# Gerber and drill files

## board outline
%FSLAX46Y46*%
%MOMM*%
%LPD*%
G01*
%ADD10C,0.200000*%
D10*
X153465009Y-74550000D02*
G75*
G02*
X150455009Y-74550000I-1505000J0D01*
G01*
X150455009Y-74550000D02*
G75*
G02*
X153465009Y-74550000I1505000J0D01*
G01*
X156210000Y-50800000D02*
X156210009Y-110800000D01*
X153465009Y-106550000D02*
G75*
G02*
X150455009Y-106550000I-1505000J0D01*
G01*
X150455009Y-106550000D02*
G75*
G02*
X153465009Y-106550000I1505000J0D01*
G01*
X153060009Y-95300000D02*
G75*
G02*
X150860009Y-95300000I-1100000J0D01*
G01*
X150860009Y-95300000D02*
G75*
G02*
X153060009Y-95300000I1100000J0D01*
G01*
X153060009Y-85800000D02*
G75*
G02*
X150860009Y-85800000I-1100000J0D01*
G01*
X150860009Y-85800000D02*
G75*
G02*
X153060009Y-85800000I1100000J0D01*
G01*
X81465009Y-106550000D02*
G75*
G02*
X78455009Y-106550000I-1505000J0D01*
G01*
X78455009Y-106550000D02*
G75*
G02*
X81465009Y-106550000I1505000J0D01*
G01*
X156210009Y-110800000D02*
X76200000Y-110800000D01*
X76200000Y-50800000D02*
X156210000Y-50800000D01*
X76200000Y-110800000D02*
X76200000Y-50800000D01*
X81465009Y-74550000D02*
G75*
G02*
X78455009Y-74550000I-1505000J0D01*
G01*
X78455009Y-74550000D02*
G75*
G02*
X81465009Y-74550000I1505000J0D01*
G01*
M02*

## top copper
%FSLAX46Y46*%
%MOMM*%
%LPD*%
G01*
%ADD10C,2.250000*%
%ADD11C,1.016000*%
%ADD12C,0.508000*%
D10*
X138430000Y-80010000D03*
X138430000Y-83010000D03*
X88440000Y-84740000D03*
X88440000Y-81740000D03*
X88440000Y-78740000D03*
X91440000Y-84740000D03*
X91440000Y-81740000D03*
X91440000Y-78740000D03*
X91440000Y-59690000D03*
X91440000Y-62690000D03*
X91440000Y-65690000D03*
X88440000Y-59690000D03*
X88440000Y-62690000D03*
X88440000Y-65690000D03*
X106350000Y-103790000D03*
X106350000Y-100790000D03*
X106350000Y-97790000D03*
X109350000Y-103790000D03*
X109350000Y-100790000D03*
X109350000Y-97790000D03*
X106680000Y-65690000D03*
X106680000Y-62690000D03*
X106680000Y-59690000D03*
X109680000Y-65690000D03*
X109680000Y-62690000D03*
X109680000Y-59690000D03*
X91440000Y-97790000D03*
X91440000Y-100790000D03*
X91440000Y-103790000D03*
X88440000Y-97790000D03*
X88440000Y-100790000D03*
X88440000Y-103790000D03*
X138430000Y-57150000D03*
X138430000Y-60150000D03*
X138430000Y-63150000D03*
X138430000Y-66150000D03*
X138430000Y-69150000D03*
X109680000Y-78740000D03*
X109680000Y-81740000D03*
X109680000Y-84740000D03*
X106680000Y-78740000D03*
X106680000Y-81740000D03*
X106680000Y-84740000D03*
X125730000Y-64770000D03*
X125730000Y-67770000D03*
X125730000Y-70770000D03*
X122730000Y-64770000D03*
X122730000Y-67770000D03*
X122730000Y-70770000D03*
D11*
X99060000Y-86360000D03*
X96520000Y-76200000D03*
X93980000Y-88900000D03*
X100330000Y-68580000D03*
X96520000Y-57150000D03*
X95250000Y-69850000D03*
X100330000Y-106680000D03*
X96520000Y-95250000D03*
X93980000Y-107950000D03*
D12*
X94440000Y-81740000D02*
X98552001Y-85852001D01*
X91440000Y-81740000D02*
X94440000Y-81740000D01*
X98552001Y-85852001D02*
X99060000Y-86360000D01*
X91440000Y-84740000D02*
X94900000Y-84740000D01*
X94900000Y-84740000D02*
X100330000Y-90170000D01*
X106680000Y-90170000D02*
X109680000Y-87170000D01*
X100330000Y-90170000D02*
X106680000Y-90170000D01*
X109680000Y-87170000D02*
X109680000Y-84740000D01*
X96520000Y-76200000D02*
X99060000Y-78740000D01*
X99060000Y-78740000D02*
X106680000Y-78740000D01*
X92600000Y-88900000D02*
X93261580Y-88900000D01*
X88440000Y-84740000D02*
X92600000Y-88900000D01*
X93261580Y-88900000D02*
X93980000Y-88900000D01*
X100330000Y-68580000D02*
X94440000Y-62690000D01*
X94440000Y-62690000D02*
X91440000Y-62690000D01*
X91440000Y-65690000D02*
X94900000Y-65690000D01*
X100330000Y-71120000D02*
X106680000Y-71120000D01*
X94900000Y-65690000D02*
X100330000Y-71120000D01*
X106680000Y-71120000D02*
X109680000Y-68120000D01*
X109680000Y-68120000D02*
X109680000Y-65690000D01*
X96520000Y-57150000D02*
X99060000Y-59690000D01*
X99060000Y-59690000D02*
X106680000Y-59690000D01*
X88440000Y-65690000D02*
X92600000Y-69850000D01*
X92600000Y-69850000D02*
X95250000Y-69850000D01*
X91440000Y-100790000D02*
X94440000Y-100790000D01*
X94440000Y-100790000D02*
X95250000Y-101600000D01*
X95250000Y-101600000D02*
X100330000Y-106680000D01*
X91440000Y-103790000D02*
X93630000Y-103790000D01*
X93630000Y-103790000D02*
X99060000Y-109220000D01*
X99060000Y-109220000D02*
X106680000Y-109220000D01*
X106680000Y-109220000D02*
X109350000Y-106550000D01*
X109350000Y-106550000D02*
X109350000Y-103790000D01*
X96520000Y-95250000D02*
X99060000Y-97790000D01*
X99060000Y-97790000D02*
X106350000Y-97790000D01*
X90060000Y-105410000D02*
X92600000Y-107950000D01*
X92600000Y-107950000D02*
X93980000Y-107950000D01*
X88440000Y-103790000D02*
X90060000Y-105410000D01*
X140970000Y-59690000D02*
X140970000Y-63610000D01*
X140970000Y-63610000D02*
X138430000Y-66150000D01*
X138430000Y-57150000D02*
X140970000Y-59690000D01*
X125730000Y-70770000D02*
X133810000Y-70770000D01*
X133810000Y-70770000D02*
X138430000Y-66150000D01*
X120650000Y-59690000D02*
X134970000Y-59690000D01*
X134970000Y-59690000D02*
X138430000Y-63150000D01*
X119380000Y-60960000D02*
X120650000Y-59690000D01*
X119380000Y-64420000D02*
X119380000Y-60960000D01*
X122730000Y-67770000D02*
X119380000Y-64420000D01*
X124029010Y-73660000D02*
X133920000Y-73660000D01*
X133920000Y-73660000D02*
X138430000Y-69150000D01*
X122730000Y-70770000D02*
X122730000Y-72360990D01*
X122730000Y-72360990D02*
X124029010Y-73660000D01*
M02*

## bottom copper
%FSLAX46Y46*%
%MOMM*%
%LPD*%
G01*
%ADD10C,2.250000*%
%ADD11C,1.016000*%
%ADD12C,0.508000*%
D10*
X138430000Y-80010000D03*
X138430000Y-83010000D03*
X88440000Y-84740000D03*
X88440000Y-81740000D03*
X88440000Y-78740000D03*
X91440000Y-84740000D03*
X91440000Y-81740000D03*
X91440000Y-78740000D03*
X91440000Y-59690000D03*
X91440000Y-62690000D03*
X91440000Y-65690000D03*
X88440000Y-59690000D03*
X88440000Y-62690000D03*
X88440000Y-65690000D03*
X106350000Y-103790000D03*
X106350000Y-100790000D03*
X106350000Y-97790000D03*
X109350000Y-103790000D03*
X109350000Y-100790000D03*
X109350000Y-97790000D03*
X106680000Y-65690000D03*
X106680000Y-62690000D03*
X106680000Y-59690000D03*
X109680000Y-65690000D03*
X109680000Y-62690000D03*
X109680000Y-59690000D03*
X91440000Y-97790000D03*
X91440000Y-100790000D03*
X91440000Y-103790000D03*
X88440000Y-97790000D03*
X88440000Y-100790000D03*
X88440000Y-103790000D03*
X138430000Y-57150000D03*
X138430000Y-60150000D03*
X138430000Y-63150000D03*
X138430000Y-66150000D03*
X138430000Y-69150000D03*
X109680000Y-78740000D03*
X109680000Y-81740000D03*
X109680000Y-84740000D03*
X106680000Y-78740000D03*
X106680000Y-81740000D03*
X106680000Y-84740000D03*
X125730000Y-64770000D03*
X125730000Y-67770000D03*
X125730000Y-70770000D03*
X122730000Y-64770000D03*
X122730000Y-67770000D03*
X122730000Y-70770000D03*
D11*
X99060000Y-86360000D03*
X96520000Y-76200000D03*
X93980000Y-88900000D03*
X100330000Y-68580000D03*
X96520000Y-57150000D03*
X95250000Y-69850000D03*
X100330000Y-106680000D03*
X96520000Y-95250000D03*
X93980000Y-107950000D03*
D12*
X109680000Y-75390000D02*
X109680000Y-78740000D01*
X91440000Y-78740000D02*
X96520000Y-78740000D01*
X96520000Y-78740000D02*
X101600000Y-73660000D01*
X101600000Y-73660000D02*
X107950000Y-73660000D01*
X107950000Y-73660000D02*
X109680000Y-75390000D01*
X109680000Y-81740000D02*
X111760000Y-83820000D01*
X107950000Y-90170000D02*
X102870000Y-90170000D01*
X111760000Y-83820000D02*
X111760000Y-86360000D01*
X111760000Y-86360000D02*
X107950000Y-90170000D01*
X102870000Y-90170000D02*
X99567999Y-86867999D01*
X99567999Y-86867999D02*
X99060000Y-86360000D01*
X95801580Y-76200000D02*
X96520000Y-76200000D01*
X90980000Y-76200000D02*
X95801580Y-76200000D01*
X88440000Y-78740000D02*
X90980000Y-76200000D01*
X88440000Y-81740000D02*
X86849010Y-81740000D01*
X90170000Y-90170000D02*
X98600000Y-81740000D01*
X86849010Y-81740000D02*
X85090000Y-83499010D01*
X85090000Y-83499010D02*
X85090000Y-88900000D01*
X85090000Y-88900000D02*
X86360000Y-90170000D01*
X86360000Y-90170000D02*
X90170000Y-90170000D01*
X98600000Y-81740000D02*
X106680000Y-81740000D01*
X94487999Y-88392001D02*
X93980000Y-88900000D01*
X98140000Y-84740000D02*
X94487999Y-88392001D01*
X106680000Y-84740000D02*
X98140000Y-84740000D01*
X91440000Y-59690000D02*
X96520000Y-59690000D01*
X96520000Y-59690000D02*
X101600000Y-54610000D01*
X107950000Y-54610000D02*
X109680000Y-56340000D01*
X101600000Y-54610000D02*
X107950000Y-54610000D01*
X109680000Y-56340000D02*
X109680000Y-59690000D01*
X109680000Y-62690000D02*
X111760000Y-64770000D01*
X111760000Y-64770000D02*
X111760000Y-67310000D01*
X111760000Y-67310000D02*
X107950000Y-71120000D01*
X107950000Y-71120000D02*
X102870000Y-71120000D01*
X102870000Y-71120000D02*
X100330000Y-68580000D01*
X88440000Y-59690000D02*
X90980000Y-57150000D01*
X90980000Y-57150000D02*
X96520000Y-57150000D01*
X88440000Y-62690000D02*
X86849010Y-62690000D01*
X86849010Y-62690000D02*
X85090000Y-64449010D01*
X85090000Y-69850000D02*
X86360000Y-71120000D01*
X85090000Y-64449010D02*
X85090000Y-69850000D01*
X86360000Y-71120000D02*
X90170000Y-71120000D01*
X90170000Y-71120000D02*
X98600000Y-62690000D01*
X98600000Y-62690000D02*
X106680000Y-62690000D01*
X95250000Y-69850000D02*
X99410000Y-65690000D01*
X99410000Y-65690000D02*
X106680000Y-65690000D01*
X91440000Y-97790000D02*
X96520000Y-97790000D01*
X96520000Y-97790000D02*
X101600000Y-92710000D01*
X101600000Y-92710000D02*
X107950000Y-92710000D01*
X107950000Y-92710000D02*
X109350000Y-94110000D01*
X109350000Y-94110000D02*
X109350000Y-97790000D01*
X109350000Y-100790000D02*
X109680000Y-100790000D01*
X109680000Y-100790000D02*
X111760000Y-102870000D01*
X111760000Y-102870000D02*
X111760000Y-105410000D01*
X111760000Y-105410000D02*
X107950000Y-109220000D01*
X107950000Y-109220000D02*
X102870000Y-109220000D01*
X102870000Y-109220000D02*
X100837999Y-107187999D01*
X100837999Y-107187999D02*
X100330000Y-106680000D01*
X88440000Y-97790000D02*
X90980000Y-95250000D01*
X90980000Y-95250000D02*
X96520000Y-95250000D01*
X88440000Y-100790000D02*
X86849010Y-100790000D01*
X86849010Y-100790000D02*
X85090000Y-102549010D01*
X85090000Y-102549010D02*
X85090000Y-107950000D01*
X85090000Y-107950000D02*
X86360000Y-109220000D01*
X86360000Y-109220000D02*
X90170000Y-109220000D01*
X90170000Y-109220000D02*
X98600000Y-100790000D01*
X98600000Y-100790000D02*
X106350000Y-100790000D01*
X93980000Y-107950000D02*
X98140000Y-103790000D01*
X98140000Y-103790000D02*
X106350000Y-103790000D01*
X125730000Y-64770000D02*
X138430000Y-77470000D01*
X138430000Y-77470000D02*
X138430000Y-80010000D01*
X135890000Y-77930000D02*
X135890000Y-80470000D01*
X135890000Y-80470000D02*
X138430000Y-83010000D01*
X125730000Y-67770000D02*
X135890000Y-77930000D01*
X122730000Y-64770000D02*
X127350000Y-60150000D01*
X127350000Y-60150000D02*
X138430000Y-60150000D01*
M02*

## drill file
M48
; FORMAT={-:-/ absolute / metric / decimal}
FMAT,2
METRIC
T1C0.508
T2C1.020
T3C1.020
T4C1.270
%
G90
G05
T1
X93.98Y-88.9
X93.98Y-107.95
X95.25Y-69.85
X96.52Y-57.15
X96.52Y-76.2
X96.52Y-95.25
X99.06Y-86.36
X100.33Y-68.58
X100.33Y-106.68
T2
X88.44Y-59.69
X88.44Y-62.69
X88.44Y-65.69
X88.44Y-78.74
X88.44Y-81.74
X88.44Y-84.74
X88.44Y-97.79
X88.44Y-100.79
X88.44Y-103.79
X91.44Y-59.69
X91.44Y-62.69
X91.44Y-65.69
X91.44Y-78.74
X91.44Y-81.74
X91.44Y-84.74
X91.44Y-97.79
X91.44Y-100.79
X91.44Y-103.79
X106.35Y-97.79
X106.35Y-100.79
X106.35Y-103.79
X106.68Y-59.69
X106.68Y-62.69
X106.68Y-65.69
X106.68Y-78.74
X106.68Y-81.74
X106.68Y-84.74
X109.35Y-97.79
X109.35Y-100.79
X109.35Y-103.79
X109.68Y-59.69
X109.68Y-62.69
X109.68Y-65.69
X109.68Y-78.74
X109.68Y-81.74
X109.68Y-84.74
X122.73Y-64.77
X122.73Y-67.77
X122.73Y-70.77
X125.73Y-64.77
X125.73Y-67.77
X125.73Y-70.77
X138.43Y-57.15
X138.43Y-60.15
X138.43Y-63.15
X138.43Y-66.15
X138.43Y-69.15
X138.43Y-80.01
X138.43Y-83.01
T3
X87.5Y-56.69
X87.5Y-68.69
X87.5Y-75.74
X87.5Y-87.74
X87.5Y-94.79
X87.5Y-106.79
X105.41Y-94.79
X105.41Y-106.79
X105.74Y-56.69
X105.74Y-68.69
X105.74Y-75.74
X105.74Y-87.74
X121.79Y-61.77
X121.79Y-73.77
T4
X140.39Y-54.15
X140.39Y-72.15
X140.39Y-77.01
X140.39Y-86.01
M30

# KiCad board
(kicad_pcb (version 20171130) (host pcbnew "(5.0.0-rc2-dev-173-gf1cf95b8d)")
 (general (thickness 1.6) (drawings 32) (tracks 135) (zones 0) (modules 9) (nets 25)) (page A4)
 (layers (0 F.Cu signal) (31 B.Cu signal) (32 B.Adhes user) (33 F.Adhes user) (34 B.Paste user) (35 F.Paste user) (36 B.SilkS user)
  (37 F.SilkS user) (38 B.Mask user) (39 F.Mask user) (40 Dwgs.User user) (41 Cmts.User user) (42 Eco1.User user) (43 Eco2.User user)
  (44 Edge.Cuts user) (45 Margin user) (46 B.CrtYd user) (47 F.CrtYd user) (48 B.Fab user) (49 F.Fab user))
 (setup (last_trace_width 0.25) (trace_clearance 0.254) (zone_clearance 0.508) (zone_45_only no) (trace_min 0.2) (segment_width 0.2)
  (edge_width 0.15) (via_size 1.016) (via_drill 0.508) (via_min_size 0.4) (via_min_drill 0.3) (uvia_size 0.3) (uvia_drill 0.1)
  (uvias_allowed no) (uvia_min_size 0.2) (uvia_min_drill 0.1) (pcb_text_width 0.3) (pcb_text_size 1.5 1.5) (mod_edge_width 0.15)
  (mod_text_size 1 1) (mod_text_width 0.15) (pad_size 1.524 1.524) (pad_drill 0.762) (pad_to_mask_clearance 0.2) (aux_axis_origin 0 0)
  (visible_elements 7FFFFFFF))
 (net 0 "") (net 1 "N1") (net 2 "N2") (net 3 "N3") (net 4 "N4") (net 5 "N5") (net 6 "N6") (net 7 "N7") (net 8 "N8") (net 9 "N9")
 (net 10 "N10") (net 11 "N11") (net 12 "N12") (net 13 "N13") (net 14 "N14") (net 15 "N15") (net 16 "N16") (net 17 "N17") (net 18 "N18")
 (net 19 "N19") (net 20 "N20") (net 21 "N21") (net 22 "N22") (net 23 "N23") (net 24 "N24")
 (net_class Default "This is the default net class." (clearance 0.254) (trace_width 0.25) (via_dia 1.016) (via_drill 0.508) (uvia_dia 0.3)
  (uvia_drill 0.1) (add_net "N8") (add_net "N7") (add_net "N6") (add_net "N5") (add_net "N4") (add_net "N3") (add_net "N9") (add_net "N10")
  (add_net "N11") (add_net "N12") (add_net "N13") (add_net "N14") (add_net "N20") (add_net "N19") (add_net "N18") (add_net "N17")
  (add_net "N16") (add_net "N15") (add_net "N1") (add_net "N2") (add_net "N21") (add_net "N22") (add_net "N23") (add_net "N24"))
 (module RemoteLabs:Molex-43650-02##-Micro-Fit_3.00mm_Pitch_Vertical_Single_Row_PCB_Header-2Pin (layer F.Cu) (at 138.43 80.01 90)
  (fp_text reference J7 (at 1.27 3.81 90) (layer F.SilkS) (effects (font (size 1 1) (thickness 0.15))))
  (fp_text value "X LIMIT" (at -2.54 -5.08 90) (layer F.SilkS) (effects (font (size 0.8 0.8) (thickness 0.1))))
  (pad 1 thru_hole circle (at 0 0 90) (size 2.25 2.25) (drill 1.02) (layers *.Cu *.Mask F.SilkS) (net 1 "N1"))
  (pad 2 thru_hole circle (at -3 0 90) (size 2.25 2.25) (drill 1.02) (layers *.Cu *.Mask F.SilkS) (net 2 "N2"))
  (pad "" np_thru_hole circle (at 3 1.96 90) (size 1.27 1.27) (drill 1.27) (layers *.Cu *.Mask F.SilkS))
  (pad "" np_thru_hole circle (at -6 1.96 90) (size 1.27 1.27) (drill 1.27) (layers *.Cu *.Mask F.SilkS)))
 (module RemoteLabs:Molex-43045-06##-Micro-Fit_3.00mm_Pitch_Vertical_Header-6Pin (layer F.Cu) (at 91.44 78.74 90)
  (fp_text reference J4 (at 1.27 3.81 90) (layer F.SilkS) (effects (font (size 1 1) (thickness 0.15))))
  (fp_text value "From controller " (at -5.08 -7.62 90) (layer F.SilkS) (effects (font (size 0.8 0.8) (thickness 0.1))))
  (pad 6 thru_hole circle (at -6 -3 90) (size 2.25 2.25) (drill 1.02) (layers *.Cu *.Mask F.SilkS) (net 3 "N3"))
  (pad 5 thru_hole circle (at -3 -3 90) (size 2.25 2.25) (drill 1.02) (layers *.Cu *.Mask F.SilkS) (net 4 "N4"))
  (pad 4 thru_hole circle (at 0 -3 90) (size 2.25 2.25) (drill 1.02) (layers *.Cu *.Mask F.SilkS) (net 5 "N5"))
  (pad 3 thru_hole circle (at -6 0 90) (size 2.25 2.25) (drill 1.02) (layers *.Cu *.Mask F.SilkS) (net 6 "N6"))
  (pad 2 thru_hole circle (at -3 0 90) (size 2.25 2.25) (drill 1.02) (layers *.Cu *.Mask F.SilkS) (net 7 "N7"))
  (pad 1 thru_hole circle (at 0 0 90) (size 2.25 2.25) (drill 1.02) (layers *.Cu *.Mask F.SilkS) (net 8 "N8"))
  (pad "" np_thru_hole circle (at -9 -3.94 90) (size 1.02 1.02) (drill 1.02) (layers *.Cu *.Mask F.SilkS))
  (pad "" np_thru_hole circle (at 3 -3.94 90) (size 1.02 1.02) (drill 1.02) (layers *.Cu *.Mask F.SilkS)))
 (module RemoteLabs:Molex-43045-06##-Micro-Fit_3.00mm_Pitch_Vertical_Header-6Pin (layer F.Cu) (at 91.44 59.69 90)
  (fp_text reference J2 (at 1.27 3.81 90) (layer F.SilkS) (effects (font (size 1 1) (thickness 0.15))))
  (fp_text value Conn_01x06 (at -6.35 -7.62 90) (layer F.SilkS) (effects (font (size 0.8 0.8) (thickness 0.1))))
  (pad "" np_thru_hole circle (at 3 -3.94 90) (size 1.02 1.02) (drill 1.02) (layers *.Cu *.Mask F.SilkS))
  (pad "" np_thru_hole circle (at -9 -3.94 90) (size 1.02 1.02) (drill 1.02) (layers *.Cu *.Mask F.SilkS))
  (pad 1 thru_hole circle (at 0 0 90) (size 2.25 2.25) (drill 1.02) (layers *.Cu *.Mask F.SilkS) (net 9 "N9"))
  (pad 2 thru_hole circle (at -3 0 90) (size 2.25 2.25) (drill 1.02) (layers *.Cu *.Mask F.SilkS) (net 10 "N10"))
  (pad 3 thru_hole circle (at -6 0 90) (size 2.25 2.25) (drill 1.02) (layers *.Cu *.Mask F.SilkS) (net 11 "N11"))
  (pad 4 thru_hole circle (at 0 -3 90) (size 2.25 2.25) (drill 1.02) (layers *.Cu *.Mask F.SilkS) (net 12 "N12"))
  (pad 5 thru_hole circle (at -3 -3 90) (size 2.25 2.25) (drill 1.02) (layers *.Cu *.Mask F.SilkS) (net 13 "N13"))
  (pad 6 thru_hole circle (at -6 -3 90) (size 2.25 2.25) (drill 1.02) (layers *.Cu *.Mask F.SilkS) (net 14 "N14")))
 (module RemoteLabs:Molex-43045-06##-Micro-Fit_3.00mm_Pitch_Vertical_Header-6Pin (layer F.Cu) (at 109.35 97.79 90)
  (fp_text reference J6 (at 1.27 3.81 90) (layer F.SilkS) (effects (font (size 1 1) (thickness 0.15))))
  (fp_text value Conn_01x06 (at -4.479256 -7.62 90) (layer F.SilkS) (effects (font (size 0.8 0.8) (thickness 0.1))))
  (pad 6 thru_hole circle (at -6 -3 90) (size 2.25 2.25) (drill 1.02) (layers *.Cu *.Mask F.SilkS) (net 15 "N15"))
  (pad 5 thru_hole circle (at -3 -3 90) (size 2.25 2.25) (drill 1.02) (layers *.Cu *.Mask F.SilkS) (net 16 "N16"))
  (pad 4 thru_hole circle (at 0 -3 90) (size 2.25 2.25) (drill 1.02) (layers *.Cu *.Mask F.SilkS) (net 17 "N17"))
  (pad 3 thru_hole circle (at -6 0 90) (size 2.25 2.25) (drill 1.02) (layers *.Cu *.Mask F.SilkS) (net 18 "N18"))
  (pad 2 thru_hole circle (at -3 0 90) (size 2.25 2.25) (drill 1.02) (layers *.Cu *.Mask F.SilkS) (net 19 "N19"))
  (pad 1 thru_hole circle (at 0 0 90) (size 2.25 2.25) (drill 1.02) (layers *.Cu *.Mask F.SilkS) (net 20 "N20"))
  (pad "" np_thru_hole circle (at -9 -3.94 90) (size 1.02 1.02) (drill 1.02) (layers *.Cu *.Mask F.SilkS))
  (pad "" np_thru_hole circle (at 3 -3.94 90) (size 1.02 1.02) (drill 1.02) (layers *.Cu *.Mask F.SilkS)))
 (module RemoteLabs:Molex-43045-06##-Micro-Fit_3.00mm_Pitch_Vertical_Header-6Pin (layer F.Cu) (at 109.68 59.69 90)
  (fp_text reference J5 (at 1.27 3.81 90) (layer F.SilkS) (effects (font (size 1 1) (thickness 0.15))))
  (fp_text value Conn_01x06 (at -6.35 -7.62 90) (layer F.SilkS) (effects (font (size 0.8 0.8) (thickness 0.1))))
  (pad 6 thru_hole circle (at -6 -3 90) (size 2.25 2.25) (drill 1.02) (layers *.Cu *.Mask F.SilkS) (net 14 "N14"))
  (pad 5 thru_hole circle (at -3 -3 90) (size 2.25 2.25) (drill 1.02) (layers *.Cu *.Mask F.SilkS) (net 13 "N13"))
  (pad 4 thru_hole circle (at 0 -3 90) (size 2.25 2.25) (drill 1.02) (layers *.Cu *.Mask F.SilkS) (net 12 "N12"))
  (pad 3 thru_hole circle (at -6 0 90) (size 2.25 2.25) (drill 1.02) (layers *.Cu *.Mask F.SilkS) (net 11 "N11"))
  (pad 2 thru_hole circle (at -3 0 90) (size 2.25 2.25) (drill 1.02) (layers *.Cu *.Mask F.SilkS) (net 10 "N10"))
  (pad 1 thru_hole circle (at 0 0 90) (size 2.25 2.25) (drill 1.02) (layers *.Cu *.Mask F.SilkS) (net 9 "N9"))
  (pad "" np_thru_hole circle (at -9 -3.94 90) (size 1.02 1.02) (drill 1.02) (layers *.Cu *.Mask F.SilkS))
  (pad "" np_thru_hole circle (at 3 -3.94 90) (size 1.02 1.02) (drill 1.02) (layers *.Cu *.Mask F.SilkS)))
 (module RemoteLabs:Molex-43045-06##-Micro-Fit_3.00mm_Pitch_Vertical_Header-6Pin (layer F.Cu) (at 91.44 97.79 90)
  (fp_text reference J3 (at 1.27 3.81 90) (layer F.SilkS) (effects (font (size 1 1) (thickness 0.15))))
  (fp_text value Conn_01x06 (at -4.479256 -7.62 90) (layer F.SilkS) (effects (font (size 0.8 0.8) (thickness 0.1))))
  (pad "" np_thru_hole circle (at 3 -3.94 90) (size 1.02 1.02) (drill 1.02) (layers *.Cu *.Mask F.SilkS))
  (pad "" np_thru_hole circle (at -9 -3.94 90) (size 1.02 1.02) (drill 1.02) (layers *.Cu *.Mask F.SilkS))
  (pad 1 thru_hole circle (at 0 0 90) (size 2.25 2.25) (drill 1.02) (layers *.Cu *.Mask F.SilkS) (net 20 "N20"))
  (pad 2 thru_hole circle (at -3 0 90) (size 2.25 2.25) (drill 1.02) (layers *.Cu *.Mask F.SilkS) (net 19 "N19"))
  (pad 3 thru_hole circle (at -6 0 90) (size 2.25 2.25) (drill 1.02) (layers *.Cu *.Mask F.SilkS) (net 18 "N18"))
  (pad 4 thru_hole circle (at 0 -3 90) (size 2.25 2.25) (drill 1.02) (layers *.Cu *.Mask F.SilkS) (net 17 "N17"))
  (pad 5 thru_hole circle (at -3 -3 90) (size 2.25 2.25) (drill 1.02) (layers *.Cu *.Mask F.SilkS) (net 16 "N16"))
  (pad 6 thru_hole circle (at -6 -3 90) (size 2.25 2.25) (drill 1.02) (layers *.Cu *.Mask F.SilkS) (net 15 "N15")))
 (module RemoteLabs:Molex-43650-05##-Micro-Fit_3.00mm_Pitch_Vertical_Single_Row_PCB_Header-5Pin (layer F.Cu) (at 138.43 57.15 90)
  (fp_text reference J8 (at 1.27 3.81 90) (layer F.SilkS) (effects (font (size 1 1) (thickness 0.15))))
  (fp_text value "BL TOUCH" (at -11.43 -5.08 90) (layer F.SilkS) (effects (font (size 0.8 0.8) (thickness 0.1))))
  (pad 1 thru_hole circle (at 0 0 90) (size 2.25 2.25) (drill 1.02) (layers *.Cu *.Mask F.SilkS) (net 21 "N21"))
  (pad 2 thru_hole circle (at -3 0 90) (size 2.25 2.25) (drill 1.02) (layers *.Cu *.Mask F.SilkS) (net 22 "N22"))
  (pad 3 thru_hole circle (at -6 0 90) (size 2.25 2.25) (drill 1.02) (layers *.Cu *.Mask F.SilkS) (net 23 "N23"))
  (pad 4 thru_hole circle (at -9 0 90) (size 2.25 2.25) (drill 1.02) (layers *.Cu *.Mask F.SilkS) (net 21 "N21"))
  (pad 5 thru_hole circle (at -12 0 90) (size 2.25 2.25) (drill 1.02) (layers *.Cu *.Mask F.SilkS) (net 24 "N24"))
  (pad "" np_thru_hole circle (at 3 1.96 90) (size 1.27 1.27) (drill 1.27) (layers *.Cu *.Mask F.SilkS))
  (pad "" np_thru_hole circle (at -15 1.96 90) (size 1.27 1.27) (drill 1.27) (layers *.Cu *.Mask F.SilkS)))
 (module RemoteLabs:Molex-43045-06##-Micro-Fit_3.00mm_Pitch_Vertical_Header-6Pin (layer F.Cu) (at 109.68 78.74 90)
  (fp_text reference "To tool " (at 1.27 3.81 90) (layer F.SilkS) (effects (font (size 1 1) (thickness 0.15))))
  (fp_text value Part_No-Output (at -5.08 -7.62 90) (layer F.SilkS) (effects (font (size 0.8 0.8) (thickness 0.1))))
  (pad "" np_thru_hole circle (at 3 -3.94 90) (size 1.02 1.02) (drill 1.02) (layers *.Cu *.Mask F.SilkS))
  (pad "" np_thru_hole circle (at -9 -3.94 90) (size 1.02 1.02) (drill 1.02) (layers *.Cu *.Mask F.SilkS))
  (pad 1 thru_hole circle (at 0 0 90) (size 2.25 2.25) (drill 1.02) (layers *.Cu *.Mask F.SilkS) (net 8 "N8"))
  (pad 2 thru_hole circle (at -3 0 90) (size 2.25 2.25) (drill 1.02) (layers *.Cu *.Mask F.SilkS) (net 7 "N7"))
  (pad 3 thru_hole circle (at -6 0 90) (size 2.25 2.25) (drill 1.02) (layers *.Cu *.Mask F.SilkS) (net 6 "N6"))
  (pad 4 thru_hole circle (at 0 -3 90) (size 2.25 2.25) (drill 1.02) (layers *.Cu *.Mask F.SilkS) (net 5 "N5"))
  (pad 5 thru_hole circle (at -3 -3 90) (size 2.25 2.25) (drill 1.02) (layers *.Cu *.Mask F.SilkS) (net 4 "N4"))
  (pad 6 thru_hole circle (at -6 -3 90) (size 2.25 2.25) (drill 1.02) (layers *.Cu *.Mask F.SilkS) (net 3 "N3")))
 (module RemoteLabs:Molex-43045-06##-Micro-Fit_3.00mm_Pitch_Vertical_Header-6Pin (layer F.Cu) (at 125.73 64.77 90)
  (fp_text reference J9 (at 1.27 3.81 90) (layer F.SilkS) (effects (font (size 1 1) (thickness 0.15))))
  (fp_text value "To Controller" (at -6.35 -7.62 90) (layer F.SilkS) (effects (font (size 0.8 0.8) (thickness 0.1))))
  (pad "" np_thru_hole circle (at 3 -3.94 90) (size 1.02 1.02) (drill 1.02) (layers *.Cu *.Mask F.SilkS))
  (pad "" np_thru_hole circle (at -9 -3.94 90) (size 1.02 1.02) (drill 1.02) (layers *.Cu *.Mask F.SilkS))
  (pad 1 thru_hole circle (at 0 0 90) (size 2.25 2.25) (drill 1.02) (layers *.Cu *.Mask F.SilkS) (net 1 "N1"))
  (pad 2 thru_hole circle (at -3 0 90) (size 2.25 2.25) (drill 1.02) (layers *.Cu *.Mask F.SilkS) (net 2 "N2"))
  (pad 3 thru_hole circle (at -6 0 90) (size 2.25 2.25) (drill 1.02) (layers *.Cu *.Mask F.SilkS) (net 21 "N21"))
  (pad 4 thru_hole circle (at 0 -3 90) (size 2.25 2.25) (drill 1.02) (layers *.Cu *.Mask F.SilkS) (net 22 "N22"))
  (pad 5 thru_hole circle (at -3 -3 90) (size 2.25 2.25) (drill 1.02) (layers *.Cu *.Mask F.SilkS) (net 23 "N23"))
  (pad 6 thru_hole circle (at -6 -3 90) (size 2.25 2.25) (drill 1.02) (layers *.Cu *.Mask F.SilkS) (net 24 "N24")))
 (gr_circle (center 151.960009 74.55) (end 153.465009 74.55) (layer Edge.Cuts) (width 0.2))
 (gr_line (start 156.21 50.8) (end 156.210009 110.8) (layer Edge.Cuts) (width 0.2))
 (gr_circle (center 151.960009 106.55) (end 153.465009 106.55) (layer Edge.Cuts) (width 0.2))
 (gr_circle (center 151.960009 95.3) (end 153.060009 95.3) (layer Edge.Cuts) (width 0.2))
 (gr_circle (center 151.960009 85.8) (end 153.060009 85.8) (layer Edge.Cuts) (width 0.2))
 (gr_circle (center 79.960009 106.55) (end 81.465009 106.55) (layer Edge.Cuts) (width 0.2))
 (gr_line (start 156.210009 110.8) (end 76.2 110.8) (layer Edge.Cuts) (width 0.2))
 (gr_line (start 76.2 50.8) (end 156.21 50.8) (layer Edge.Cuts) (width 0.2))
 (gr_line (start 76.2 110.8) (end 76.2 50.8) (layer Edge.Cuts) (width 0.2))
 (gr_circle (center 79.960009 74.55) (end 81.465009 74.55) (layer Edge.Cuts) (width 0.2))
 (segment (start 109.68 75.39) (end 109.68 78.74) (width 0.508) (layer B.Cu) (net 8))
 (segment (start 91.44 78.74) (end 96.52 78.74) (width 0.508) (layer B.Cu) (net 8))
 (segment (start 96.52 78.74) (end 101.6 73.66) (width 0.508) (layer B.Cu) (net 8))
 (segment (start 101.6 73.66) (end 107.95 73.66) (width 0.508) (layer B.Cu) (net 8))
 (segment (start 107.95 73.66) (end 109.68 75.39) (width 0.508) (layer B.Cu) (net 8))
 (segment (start 109.68 81.74) (end 111.76 83.82) (width 0.508) (layer B.Cu) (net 7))
 (segment (start 107.95 90.17) (end 102.87 90.17) (width 0.508) (layer B.Cu) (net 7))
 (segment (start 111.76 83.82) (end 111.76 86.36) (width 0.508) (layer B.Cu) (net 7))
 (segment (start 111.76 86.36) (end 107.95 90.17) (width 0.508) (layer B.Cu) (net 7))
 (segment (start 102.87 90.17) (end 99.567999 86.867999) (width 0.508) (layer B.Cu) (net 7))
 (segment (start 99.567999 86.867999) (end 99.06 86.36) (width 0.508) (layer B.Cu) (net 7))
 (segment (start 94.44 81.74) (end 98.552001 85.852001) (width 0.508) (layer F.Cu) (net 7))
 (segment (start 91.44 81.74) (end 94.44 81.74) (width 0.508) (layer F.Cu) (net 7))
 (segment (start 98.552001 85.852001) (end 99.06 86.36) (width 0.508) (layer F.Cu) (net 7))
 (via (at 99.06 86.36) (size 1.016) (drill 0.508) (layers F.Cu B.Cu) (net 7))
 (segment (start 91.44 84.74) (end 94.9 84.74) (width 0.508) (layer F.Cu) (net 6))
 (segment (start 94.9 84.74) (end 100.33 90.17) (width 0.508) (layer F.Cu) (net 6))
 (segment (start 106.68 90.17) (end 109.68 87.17) (width 0.508) (layer F.Cu) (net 6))
 (segment (start 100.33 90.17) (end 106.68 90.17) (width 0.508) (layer F.Cu) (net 6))
 (segment (start 109.68 87.17) (end 109.68 84.74) (width 0.508) (layer F.Cu) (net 6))
 (segment (start 96.52 76.2) (end 99.06 78.74) (width 0.508) (layer F.Cu) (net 5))
 (segment (start 99.06 78.74) (end 106.68 78.74) (width 0.508) (layer F.Cu) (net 5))
 (segment (start 95.80158 76.2) (end 96.52 76.2) (width 0.508) (layer B.Cu) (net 5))
 (segment (start 90.98 76.2) (end 95.80158 76.2) (width 0.508) (layer B.Cu) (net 5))
 (segment (start 88.44 78.74) (end 90.98 76.2) (width 0.508) (layer B.Cu) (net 5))
 (via (at 96.52 76.2) (size 1.016) (drill 0.508) (layers F.Cu B.Cu) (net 5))
 (segment (start 88.44 81.74) (end 86.84901 81.74) (width 0.508) (layer B.Cu) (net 4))
 (segment (start 90.17 90.17) (end 98.6 81.74) (width 0.508) (layer B.Cu) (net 4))
 (segment (start 86.84901 81.74) (end 85.09 83.49901) (width 0.508) (layer B.Cu) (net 4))
 (segment (start 85.09 83.49901) (end 85.09 88.9) (width 0.508) (layer B.Cu) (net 4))
 (segment (start 85.09 88.9) (end 86.36 90.17) (width 0.508) (layer B.Cu) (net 4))
 (segment (start 86.36 90.17) (end 90.17 90.17) (width 0.508) (layer B.Cu) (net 4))
 (segment (start 98.6 81.74) (end 106.68 81.74) (width 0.508) (layer B.Cu) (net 4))
 (segment (start 92.6 88.9) (end 93.26158 88.9) (width 0.508) (layer F.Cu) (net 3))
 (segment (start 88.44 84.74) (end 92.6 88.9) (width 0.508) (layer F.Cu) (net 3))
 (segment (start 93.26158 88.9) (end 93.98 88.9) (width 0.508) (layer F.Cu) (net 3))
 (segment (start 94.487999 88.392001) (end 93.98 88.9) (width 0.508) (layer B.Cu) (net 3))
 (segment (start 98.14 84.74) (end 94.487999 88.392001) (width 0.508) (layer B.Cu) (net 3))
 (segment (start 106.68 84.74) (end 98.14 84.74) (width 0.508) (layer B.Cu) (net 3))
 (via (at 93.98 88.9) (size 1.016) (drill 0.508) (layers F.Cu B.Cu) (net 3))
 (segment (start 91.44 59.69) (end 96.52 59.69) (width 0.508) (layer B.Cu) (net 9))
 (segment (start 96.52 59.69) (end 101.6 54.61) (width 0.508) (layer B.Cu) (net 9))
 (segment (start 107.95 54.61) (end 109.68 56.34) (width 0.508) (layer B.Cu) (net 9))
 (segment (start 101.6 54.61) (end 107.95 54.61) (width 0.508) (layer B.Cu) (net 9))
 (segment (start 109.68 56.34) (end 109.68 59.69) (width 0.508) (layer B.Cu) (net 9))
 (segment (start 109.68 62.69) (end 111.76 64.77) (width 0.508) (layer B.Cu) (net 10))
 (segment (start 111.76 64.77) (end 111.76 67.31) (width 0.508) (layer B.Cu) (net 10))
 (segment (start 111.76 67.31) (end 107.95 71.12) (width 0.508) (layer B.Cu) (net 10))
 (segment (start 107.95 71.12) (end 102.87 71.12) (width 0.508) (layer B.Cu) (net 10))
 (segment (start 102.87 71.12) (end 100.33 68.58) (width 0.508) (layer B.Cu) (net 10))
 (segment (start 100.33 68.58) (end 94.44 62.69) (width 0.508) (layer F.Cu) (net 10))
 (segment (start 94.44 62.69) (end 91.44 62.69) (width 0.508) (layer F.Cu) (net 10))
 (via (at 100.33 68.58) (size 1.016) (drill 0.508) (layers F.Cu B.Cu) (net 10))
 (segment (start 91.44 65.69) (end 94.9 65.69) (width 0.508) (layer F.Cu) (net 11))
 (segment (start 100.33 71.12) (end 106.68 71.12) (width 0.508) (layer F.Cu) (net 11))
 (segment (start 94.9 65.69) (end 100.33 71.12) (width 0.508) (layer F.Cu) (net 11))
 (segment (start 106.68 71.12) (end 109.68 68.12) (width 0.508) (layer F.Cu) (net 11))
 (segment (start 109.68 68.12) (end 109.68 65.69) (width 0.508) (layer F.Cu) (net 11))
 (segment (start 96.52 57.15) (end 99.06 59.69) (width 0.508) (layer F.Cu) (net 12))
 (segment (start 99.06 59.69) (end 106.68 59.69) (width 0.508) (layer F.Cu) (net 12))
 (segment (start 88.44 59.69) (end 90.98 57.15) (width 0.508) (layer B.Cu) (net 12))
 (segment (start 90.98 57.15) (end 96.52 57.15) (width 0.508) (layer B.Cu) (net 12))
 (via (at 96.52 57.15) (size 1.016) (drill 0.508) (layers F.Cu B.Cu) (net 12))
 (segment (start 88.44 62.69) (end 86.84901 62.69) (width 0.508) (layer B.Cu) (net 13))
 (segment (start 86.84901 62.69) (end 85.09 64.44901) (width 0.508) (layer B.Cu) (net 13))
 (segment (start 85.09 69.85) (end 86.36 71.12) (width 0.508) (layer B.Cu) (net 13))
 (segment (start 85.09 64.44901) (end 85.09 69.85) (width 0.508) (layer B.Cu) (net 13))
 (segment (start 86.36 71.12) (end 90.17 71.12) (width 0.508) (layer B.Cu) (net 13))
 (segment (start 90.17 71.12) (end 98.6 62.69) (width 0.508) (layer B.Cu) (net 13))
 (segment (start 98.6 62.69) (end 106.68 62.69) (width 0.508) (layer B.Cu) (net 13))
 (segment (start 95.25 69.85) (end 99.41 65.69) (width 0.508) (layer B.Cu) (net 14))
 (segment (start 99.41 65.69) (end 106.68 65.69) (width 0.508) (layer B.Cu) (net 14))
 (segment (start 88.44 65.69) (end 92.6 69.85) (width 0.508) (layer F.Cu) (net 14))
 (segment (start 92.6 69.85) (end 95.25 69.85) (width 0.508) (layer F.Cu) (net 14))
 (via (at 95.25 69.85) (size 1.016) (drill 0.508) (layers F.Cu B.Cu) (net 14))
 (segment (start 91.44 97.79) (end 96.52 97.79) (width 0.508) (layer B.Cu) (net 20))
 (segment (start 96.52 97.79) (end 101.6 92.71) (width 0.508) (layer B.Cu) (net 20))
 (segment (start 101.6 92.71) (end 107.95 92.71) (width 0.508) (layer B.Cu) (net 20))
 (segment (start 107.95 92.71) (end 109.35 94.11) (width 0.508) (layer B.Cu) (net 20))
 (segment (start 109.35 94.11) (end 109.35 97.79) (width 0.508) (layer B.Cu) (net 20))
 (segment (start 109.35 100.79) (end 109.68 100.79) (width 0.508) (layer B.Cu) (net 19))
 (segment (start 109.68 100.79) (end 111.76 102.87) (width 0.508) (layer B.Cu) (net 19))
 (segment (start 111.76 102.87) (end 111.76 105.41) (width 0.508) (layer B.Cu) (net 19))
 (segment (start 111.76 105.41) (end 107.95 109.22) (width 0.508) (layer B.Cu) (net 19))
 (segment (start 107.95 109.22) (end 102.87 109.22) (width 0.508) (layer B.Cu) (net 19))
 (segment (start 102.87 109.22) (end 100.837999 107.187999) (width 0.508) (layer B.Cu) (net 19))
 (segment (start 100.837999 107.187999) (end 100.33 106.68) (width 0.508) (layer B.Cu) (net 19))
 (segment (start 91.44 100.79) (end 94.44 100.79) (width 0.508) (layer F.Cu) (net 19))
 (segment (start 94.44 100.79) (end 95.25 101.6) (width 0.508) (layer F.Cu) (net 19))
 (segment (start 95.25 101.6) (end 100.33 106.68) (width 0.508) (layer F.Cu) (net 19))
 (via (at 100.33 106.68) (size 1.016) (drill 0.508) (layers F.Cu B.Cu) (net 19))
 (segment (start 91.44 103.79) (end 93.63 103.79) (width 0.508) (layer F.Cu) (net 18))
 (segment (start 93.63 103.79) (end 99.06 109.22) (width 0.508) (layer F.Cu) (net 18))
 (segment (start 99.06 109.22) (end 106.68 109.22) (width 0.508) (layer F.Cu) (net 18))
 (segment (start 106.68 109.22) (end 109.35 106.55) (width 0.508) (layer F.Cu) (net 18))
 (segment (start 109.35 106.55) (end 109.35 103.79) (width 0.508) (layer F.Cu) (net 18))
 (segment (start 96.52 95.25) (end 99.06 97.79) (width 0.508) (layer F.Cu) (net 17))
 (segment (start 99.06 97.79) (end 106.35 97.79) (width 0.508) (layer F.Cu) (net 17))
 (segment (start 88.44 97.79) (end 90.98 95.25) (width 0.508) (layer B.Cu) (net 17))
 (segment (start 90.98 95.25) (end 96.52 95.25) (width 0.508) (layer B.Cu) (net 17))
 (via (at 96.52 95.25) (size 1.016) (drill 0.508) (layers F.Cu B.Cu) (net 17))
 (segment (start 88.44 100.79) (end 86.84901 100.79) (width 0.508) (layer B.Cu) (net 16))
 (segment (start 86.84901 100.79) (end 85.09 102.54901) (width 0.508) (layer B.Cu) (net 16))
 (segment (start 85.09 102.54901) (end 85.09 107.95) (width 0.508) (layer B.Cu) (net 16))
 (segment (start 85.09 107.95) (end 86.36 109.22) (width 0.508) (layer B.Cu) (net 16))
 (segment (start 86.36 109.22) (end 90.17 109.22) (width 0.508) (layer B.Cu) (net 16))
 (segment (start 90.17 109.22) (end 98.6 100.79) (width 0.508) (layer B.Cu) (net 16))
 (segment (start 98.6 100.79) (end 106.35 100.79) (width 0.508) (layer B.Cu) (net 16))
 (segment (start 93.98 107.95) (end 98.14 103.79) (width 0.508) (layer B.Cu) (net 15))
 (segment (start 98.14 103.79) (end 106.35 103.79) (width 0.508) (layer B.Cu) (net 15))
 (segment (start 90.06 105.41) (end 92.6 107.95) (width 0.508) (layer F.Cu) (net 15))
 (segment (start 92.6 107.95) (end 93.98 107.95) (width 0.508) (layer F.Cu) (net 15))
 (via (at 93.98 107.95) (size 1.016) (drill 0.508) (layers F.Cu B.Cu) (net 15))
 (segment (start 88.44 103.79) (end 90.06 105.41) (width 0.508) (layer F.Cu) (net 15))
 (segment (start 125.73 64.77) (end 138.43 77.47) (width 0.508) (layer B.Cu) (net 1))
 (segment (start 138.43 77.47) (end 138.43 80.01) (width 0.508) (layer B.Cu) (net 1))
 (segment (start 135.89 77.93) (end 135.89 80.47) (width 0.508) (layer B.Cu) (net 2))
 (segment (start 135.89 80.47) (end 138.43 83.01) (width 0.508) (layer B.Cu) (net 2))
 (segment (start 125.73 67.77) (end 135.89 77.93) (width 0.508) (layer B.Cu) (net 2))
 (segment (start 140.97 59.69) (end 140.97 63.61) (width 0.508) (layer F.Cu) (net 21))
 (segment (start 140.97 63.61) (end 138.43 66.15) (width 0.508) (layer F.Cu) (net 21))
 (segment (start 138.43 57.15) (end 140.97 59.69) (width 0.508) (layer F.Cu) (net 21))
 (segment (start 125.73 70.77) (end 133.81 70.77) (width 0.508) (layer F.Cu) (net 21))
 (segment (start 133.81 70.77) (end 138.43 66.15) (width 0.508) (layer F.Cu) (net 21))
 (segment (start 122.73 64.77) (end 127.35 60.15) (width 0.508) (layer B.Cu) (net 22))
 (segment (start 127.35 60.15) (end 138.43 60.15) (width 0.508) (layer B.Cu) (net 22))
 (segment (start 120.65 59.69) (end 134.97 59.69) (width 0.508) (layer F.Cu) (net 23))
 (segment (start 134.97 59.69) (end 138.43 63.15) (width 0.508) (layer F.Cu) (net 23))
 (segment (start 119.38 60.96) (end 120.65 59.69) (width 0.508) (layer F.Cu) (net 23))
 (segment (start 119.38 64.42) (end 119.38 60.96) (width 0.508) (layer F.Cu) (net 23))
 (segment (start 122.73 67.77) (end 119.38 64.42) (width 0.508) (layer F.Cu) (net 23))
 (segment (start 124.02901 73.66) (end 133.92 73.66) (width 0.508) (layer F.Cu) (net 24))
 (segment (start 133.92 73.66) (end 138.43 69.15) (width 0.508) (layer F.Cu) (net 24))
 (segment (start 122.73 70.77) (end 122.73 72.36099) (width 0.508) (layer F.Cu) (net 24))
 (segment (start 122.73 72.36099) (end 124.02901 73.66) (width 0.508) (layer F.Cu) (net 24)))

